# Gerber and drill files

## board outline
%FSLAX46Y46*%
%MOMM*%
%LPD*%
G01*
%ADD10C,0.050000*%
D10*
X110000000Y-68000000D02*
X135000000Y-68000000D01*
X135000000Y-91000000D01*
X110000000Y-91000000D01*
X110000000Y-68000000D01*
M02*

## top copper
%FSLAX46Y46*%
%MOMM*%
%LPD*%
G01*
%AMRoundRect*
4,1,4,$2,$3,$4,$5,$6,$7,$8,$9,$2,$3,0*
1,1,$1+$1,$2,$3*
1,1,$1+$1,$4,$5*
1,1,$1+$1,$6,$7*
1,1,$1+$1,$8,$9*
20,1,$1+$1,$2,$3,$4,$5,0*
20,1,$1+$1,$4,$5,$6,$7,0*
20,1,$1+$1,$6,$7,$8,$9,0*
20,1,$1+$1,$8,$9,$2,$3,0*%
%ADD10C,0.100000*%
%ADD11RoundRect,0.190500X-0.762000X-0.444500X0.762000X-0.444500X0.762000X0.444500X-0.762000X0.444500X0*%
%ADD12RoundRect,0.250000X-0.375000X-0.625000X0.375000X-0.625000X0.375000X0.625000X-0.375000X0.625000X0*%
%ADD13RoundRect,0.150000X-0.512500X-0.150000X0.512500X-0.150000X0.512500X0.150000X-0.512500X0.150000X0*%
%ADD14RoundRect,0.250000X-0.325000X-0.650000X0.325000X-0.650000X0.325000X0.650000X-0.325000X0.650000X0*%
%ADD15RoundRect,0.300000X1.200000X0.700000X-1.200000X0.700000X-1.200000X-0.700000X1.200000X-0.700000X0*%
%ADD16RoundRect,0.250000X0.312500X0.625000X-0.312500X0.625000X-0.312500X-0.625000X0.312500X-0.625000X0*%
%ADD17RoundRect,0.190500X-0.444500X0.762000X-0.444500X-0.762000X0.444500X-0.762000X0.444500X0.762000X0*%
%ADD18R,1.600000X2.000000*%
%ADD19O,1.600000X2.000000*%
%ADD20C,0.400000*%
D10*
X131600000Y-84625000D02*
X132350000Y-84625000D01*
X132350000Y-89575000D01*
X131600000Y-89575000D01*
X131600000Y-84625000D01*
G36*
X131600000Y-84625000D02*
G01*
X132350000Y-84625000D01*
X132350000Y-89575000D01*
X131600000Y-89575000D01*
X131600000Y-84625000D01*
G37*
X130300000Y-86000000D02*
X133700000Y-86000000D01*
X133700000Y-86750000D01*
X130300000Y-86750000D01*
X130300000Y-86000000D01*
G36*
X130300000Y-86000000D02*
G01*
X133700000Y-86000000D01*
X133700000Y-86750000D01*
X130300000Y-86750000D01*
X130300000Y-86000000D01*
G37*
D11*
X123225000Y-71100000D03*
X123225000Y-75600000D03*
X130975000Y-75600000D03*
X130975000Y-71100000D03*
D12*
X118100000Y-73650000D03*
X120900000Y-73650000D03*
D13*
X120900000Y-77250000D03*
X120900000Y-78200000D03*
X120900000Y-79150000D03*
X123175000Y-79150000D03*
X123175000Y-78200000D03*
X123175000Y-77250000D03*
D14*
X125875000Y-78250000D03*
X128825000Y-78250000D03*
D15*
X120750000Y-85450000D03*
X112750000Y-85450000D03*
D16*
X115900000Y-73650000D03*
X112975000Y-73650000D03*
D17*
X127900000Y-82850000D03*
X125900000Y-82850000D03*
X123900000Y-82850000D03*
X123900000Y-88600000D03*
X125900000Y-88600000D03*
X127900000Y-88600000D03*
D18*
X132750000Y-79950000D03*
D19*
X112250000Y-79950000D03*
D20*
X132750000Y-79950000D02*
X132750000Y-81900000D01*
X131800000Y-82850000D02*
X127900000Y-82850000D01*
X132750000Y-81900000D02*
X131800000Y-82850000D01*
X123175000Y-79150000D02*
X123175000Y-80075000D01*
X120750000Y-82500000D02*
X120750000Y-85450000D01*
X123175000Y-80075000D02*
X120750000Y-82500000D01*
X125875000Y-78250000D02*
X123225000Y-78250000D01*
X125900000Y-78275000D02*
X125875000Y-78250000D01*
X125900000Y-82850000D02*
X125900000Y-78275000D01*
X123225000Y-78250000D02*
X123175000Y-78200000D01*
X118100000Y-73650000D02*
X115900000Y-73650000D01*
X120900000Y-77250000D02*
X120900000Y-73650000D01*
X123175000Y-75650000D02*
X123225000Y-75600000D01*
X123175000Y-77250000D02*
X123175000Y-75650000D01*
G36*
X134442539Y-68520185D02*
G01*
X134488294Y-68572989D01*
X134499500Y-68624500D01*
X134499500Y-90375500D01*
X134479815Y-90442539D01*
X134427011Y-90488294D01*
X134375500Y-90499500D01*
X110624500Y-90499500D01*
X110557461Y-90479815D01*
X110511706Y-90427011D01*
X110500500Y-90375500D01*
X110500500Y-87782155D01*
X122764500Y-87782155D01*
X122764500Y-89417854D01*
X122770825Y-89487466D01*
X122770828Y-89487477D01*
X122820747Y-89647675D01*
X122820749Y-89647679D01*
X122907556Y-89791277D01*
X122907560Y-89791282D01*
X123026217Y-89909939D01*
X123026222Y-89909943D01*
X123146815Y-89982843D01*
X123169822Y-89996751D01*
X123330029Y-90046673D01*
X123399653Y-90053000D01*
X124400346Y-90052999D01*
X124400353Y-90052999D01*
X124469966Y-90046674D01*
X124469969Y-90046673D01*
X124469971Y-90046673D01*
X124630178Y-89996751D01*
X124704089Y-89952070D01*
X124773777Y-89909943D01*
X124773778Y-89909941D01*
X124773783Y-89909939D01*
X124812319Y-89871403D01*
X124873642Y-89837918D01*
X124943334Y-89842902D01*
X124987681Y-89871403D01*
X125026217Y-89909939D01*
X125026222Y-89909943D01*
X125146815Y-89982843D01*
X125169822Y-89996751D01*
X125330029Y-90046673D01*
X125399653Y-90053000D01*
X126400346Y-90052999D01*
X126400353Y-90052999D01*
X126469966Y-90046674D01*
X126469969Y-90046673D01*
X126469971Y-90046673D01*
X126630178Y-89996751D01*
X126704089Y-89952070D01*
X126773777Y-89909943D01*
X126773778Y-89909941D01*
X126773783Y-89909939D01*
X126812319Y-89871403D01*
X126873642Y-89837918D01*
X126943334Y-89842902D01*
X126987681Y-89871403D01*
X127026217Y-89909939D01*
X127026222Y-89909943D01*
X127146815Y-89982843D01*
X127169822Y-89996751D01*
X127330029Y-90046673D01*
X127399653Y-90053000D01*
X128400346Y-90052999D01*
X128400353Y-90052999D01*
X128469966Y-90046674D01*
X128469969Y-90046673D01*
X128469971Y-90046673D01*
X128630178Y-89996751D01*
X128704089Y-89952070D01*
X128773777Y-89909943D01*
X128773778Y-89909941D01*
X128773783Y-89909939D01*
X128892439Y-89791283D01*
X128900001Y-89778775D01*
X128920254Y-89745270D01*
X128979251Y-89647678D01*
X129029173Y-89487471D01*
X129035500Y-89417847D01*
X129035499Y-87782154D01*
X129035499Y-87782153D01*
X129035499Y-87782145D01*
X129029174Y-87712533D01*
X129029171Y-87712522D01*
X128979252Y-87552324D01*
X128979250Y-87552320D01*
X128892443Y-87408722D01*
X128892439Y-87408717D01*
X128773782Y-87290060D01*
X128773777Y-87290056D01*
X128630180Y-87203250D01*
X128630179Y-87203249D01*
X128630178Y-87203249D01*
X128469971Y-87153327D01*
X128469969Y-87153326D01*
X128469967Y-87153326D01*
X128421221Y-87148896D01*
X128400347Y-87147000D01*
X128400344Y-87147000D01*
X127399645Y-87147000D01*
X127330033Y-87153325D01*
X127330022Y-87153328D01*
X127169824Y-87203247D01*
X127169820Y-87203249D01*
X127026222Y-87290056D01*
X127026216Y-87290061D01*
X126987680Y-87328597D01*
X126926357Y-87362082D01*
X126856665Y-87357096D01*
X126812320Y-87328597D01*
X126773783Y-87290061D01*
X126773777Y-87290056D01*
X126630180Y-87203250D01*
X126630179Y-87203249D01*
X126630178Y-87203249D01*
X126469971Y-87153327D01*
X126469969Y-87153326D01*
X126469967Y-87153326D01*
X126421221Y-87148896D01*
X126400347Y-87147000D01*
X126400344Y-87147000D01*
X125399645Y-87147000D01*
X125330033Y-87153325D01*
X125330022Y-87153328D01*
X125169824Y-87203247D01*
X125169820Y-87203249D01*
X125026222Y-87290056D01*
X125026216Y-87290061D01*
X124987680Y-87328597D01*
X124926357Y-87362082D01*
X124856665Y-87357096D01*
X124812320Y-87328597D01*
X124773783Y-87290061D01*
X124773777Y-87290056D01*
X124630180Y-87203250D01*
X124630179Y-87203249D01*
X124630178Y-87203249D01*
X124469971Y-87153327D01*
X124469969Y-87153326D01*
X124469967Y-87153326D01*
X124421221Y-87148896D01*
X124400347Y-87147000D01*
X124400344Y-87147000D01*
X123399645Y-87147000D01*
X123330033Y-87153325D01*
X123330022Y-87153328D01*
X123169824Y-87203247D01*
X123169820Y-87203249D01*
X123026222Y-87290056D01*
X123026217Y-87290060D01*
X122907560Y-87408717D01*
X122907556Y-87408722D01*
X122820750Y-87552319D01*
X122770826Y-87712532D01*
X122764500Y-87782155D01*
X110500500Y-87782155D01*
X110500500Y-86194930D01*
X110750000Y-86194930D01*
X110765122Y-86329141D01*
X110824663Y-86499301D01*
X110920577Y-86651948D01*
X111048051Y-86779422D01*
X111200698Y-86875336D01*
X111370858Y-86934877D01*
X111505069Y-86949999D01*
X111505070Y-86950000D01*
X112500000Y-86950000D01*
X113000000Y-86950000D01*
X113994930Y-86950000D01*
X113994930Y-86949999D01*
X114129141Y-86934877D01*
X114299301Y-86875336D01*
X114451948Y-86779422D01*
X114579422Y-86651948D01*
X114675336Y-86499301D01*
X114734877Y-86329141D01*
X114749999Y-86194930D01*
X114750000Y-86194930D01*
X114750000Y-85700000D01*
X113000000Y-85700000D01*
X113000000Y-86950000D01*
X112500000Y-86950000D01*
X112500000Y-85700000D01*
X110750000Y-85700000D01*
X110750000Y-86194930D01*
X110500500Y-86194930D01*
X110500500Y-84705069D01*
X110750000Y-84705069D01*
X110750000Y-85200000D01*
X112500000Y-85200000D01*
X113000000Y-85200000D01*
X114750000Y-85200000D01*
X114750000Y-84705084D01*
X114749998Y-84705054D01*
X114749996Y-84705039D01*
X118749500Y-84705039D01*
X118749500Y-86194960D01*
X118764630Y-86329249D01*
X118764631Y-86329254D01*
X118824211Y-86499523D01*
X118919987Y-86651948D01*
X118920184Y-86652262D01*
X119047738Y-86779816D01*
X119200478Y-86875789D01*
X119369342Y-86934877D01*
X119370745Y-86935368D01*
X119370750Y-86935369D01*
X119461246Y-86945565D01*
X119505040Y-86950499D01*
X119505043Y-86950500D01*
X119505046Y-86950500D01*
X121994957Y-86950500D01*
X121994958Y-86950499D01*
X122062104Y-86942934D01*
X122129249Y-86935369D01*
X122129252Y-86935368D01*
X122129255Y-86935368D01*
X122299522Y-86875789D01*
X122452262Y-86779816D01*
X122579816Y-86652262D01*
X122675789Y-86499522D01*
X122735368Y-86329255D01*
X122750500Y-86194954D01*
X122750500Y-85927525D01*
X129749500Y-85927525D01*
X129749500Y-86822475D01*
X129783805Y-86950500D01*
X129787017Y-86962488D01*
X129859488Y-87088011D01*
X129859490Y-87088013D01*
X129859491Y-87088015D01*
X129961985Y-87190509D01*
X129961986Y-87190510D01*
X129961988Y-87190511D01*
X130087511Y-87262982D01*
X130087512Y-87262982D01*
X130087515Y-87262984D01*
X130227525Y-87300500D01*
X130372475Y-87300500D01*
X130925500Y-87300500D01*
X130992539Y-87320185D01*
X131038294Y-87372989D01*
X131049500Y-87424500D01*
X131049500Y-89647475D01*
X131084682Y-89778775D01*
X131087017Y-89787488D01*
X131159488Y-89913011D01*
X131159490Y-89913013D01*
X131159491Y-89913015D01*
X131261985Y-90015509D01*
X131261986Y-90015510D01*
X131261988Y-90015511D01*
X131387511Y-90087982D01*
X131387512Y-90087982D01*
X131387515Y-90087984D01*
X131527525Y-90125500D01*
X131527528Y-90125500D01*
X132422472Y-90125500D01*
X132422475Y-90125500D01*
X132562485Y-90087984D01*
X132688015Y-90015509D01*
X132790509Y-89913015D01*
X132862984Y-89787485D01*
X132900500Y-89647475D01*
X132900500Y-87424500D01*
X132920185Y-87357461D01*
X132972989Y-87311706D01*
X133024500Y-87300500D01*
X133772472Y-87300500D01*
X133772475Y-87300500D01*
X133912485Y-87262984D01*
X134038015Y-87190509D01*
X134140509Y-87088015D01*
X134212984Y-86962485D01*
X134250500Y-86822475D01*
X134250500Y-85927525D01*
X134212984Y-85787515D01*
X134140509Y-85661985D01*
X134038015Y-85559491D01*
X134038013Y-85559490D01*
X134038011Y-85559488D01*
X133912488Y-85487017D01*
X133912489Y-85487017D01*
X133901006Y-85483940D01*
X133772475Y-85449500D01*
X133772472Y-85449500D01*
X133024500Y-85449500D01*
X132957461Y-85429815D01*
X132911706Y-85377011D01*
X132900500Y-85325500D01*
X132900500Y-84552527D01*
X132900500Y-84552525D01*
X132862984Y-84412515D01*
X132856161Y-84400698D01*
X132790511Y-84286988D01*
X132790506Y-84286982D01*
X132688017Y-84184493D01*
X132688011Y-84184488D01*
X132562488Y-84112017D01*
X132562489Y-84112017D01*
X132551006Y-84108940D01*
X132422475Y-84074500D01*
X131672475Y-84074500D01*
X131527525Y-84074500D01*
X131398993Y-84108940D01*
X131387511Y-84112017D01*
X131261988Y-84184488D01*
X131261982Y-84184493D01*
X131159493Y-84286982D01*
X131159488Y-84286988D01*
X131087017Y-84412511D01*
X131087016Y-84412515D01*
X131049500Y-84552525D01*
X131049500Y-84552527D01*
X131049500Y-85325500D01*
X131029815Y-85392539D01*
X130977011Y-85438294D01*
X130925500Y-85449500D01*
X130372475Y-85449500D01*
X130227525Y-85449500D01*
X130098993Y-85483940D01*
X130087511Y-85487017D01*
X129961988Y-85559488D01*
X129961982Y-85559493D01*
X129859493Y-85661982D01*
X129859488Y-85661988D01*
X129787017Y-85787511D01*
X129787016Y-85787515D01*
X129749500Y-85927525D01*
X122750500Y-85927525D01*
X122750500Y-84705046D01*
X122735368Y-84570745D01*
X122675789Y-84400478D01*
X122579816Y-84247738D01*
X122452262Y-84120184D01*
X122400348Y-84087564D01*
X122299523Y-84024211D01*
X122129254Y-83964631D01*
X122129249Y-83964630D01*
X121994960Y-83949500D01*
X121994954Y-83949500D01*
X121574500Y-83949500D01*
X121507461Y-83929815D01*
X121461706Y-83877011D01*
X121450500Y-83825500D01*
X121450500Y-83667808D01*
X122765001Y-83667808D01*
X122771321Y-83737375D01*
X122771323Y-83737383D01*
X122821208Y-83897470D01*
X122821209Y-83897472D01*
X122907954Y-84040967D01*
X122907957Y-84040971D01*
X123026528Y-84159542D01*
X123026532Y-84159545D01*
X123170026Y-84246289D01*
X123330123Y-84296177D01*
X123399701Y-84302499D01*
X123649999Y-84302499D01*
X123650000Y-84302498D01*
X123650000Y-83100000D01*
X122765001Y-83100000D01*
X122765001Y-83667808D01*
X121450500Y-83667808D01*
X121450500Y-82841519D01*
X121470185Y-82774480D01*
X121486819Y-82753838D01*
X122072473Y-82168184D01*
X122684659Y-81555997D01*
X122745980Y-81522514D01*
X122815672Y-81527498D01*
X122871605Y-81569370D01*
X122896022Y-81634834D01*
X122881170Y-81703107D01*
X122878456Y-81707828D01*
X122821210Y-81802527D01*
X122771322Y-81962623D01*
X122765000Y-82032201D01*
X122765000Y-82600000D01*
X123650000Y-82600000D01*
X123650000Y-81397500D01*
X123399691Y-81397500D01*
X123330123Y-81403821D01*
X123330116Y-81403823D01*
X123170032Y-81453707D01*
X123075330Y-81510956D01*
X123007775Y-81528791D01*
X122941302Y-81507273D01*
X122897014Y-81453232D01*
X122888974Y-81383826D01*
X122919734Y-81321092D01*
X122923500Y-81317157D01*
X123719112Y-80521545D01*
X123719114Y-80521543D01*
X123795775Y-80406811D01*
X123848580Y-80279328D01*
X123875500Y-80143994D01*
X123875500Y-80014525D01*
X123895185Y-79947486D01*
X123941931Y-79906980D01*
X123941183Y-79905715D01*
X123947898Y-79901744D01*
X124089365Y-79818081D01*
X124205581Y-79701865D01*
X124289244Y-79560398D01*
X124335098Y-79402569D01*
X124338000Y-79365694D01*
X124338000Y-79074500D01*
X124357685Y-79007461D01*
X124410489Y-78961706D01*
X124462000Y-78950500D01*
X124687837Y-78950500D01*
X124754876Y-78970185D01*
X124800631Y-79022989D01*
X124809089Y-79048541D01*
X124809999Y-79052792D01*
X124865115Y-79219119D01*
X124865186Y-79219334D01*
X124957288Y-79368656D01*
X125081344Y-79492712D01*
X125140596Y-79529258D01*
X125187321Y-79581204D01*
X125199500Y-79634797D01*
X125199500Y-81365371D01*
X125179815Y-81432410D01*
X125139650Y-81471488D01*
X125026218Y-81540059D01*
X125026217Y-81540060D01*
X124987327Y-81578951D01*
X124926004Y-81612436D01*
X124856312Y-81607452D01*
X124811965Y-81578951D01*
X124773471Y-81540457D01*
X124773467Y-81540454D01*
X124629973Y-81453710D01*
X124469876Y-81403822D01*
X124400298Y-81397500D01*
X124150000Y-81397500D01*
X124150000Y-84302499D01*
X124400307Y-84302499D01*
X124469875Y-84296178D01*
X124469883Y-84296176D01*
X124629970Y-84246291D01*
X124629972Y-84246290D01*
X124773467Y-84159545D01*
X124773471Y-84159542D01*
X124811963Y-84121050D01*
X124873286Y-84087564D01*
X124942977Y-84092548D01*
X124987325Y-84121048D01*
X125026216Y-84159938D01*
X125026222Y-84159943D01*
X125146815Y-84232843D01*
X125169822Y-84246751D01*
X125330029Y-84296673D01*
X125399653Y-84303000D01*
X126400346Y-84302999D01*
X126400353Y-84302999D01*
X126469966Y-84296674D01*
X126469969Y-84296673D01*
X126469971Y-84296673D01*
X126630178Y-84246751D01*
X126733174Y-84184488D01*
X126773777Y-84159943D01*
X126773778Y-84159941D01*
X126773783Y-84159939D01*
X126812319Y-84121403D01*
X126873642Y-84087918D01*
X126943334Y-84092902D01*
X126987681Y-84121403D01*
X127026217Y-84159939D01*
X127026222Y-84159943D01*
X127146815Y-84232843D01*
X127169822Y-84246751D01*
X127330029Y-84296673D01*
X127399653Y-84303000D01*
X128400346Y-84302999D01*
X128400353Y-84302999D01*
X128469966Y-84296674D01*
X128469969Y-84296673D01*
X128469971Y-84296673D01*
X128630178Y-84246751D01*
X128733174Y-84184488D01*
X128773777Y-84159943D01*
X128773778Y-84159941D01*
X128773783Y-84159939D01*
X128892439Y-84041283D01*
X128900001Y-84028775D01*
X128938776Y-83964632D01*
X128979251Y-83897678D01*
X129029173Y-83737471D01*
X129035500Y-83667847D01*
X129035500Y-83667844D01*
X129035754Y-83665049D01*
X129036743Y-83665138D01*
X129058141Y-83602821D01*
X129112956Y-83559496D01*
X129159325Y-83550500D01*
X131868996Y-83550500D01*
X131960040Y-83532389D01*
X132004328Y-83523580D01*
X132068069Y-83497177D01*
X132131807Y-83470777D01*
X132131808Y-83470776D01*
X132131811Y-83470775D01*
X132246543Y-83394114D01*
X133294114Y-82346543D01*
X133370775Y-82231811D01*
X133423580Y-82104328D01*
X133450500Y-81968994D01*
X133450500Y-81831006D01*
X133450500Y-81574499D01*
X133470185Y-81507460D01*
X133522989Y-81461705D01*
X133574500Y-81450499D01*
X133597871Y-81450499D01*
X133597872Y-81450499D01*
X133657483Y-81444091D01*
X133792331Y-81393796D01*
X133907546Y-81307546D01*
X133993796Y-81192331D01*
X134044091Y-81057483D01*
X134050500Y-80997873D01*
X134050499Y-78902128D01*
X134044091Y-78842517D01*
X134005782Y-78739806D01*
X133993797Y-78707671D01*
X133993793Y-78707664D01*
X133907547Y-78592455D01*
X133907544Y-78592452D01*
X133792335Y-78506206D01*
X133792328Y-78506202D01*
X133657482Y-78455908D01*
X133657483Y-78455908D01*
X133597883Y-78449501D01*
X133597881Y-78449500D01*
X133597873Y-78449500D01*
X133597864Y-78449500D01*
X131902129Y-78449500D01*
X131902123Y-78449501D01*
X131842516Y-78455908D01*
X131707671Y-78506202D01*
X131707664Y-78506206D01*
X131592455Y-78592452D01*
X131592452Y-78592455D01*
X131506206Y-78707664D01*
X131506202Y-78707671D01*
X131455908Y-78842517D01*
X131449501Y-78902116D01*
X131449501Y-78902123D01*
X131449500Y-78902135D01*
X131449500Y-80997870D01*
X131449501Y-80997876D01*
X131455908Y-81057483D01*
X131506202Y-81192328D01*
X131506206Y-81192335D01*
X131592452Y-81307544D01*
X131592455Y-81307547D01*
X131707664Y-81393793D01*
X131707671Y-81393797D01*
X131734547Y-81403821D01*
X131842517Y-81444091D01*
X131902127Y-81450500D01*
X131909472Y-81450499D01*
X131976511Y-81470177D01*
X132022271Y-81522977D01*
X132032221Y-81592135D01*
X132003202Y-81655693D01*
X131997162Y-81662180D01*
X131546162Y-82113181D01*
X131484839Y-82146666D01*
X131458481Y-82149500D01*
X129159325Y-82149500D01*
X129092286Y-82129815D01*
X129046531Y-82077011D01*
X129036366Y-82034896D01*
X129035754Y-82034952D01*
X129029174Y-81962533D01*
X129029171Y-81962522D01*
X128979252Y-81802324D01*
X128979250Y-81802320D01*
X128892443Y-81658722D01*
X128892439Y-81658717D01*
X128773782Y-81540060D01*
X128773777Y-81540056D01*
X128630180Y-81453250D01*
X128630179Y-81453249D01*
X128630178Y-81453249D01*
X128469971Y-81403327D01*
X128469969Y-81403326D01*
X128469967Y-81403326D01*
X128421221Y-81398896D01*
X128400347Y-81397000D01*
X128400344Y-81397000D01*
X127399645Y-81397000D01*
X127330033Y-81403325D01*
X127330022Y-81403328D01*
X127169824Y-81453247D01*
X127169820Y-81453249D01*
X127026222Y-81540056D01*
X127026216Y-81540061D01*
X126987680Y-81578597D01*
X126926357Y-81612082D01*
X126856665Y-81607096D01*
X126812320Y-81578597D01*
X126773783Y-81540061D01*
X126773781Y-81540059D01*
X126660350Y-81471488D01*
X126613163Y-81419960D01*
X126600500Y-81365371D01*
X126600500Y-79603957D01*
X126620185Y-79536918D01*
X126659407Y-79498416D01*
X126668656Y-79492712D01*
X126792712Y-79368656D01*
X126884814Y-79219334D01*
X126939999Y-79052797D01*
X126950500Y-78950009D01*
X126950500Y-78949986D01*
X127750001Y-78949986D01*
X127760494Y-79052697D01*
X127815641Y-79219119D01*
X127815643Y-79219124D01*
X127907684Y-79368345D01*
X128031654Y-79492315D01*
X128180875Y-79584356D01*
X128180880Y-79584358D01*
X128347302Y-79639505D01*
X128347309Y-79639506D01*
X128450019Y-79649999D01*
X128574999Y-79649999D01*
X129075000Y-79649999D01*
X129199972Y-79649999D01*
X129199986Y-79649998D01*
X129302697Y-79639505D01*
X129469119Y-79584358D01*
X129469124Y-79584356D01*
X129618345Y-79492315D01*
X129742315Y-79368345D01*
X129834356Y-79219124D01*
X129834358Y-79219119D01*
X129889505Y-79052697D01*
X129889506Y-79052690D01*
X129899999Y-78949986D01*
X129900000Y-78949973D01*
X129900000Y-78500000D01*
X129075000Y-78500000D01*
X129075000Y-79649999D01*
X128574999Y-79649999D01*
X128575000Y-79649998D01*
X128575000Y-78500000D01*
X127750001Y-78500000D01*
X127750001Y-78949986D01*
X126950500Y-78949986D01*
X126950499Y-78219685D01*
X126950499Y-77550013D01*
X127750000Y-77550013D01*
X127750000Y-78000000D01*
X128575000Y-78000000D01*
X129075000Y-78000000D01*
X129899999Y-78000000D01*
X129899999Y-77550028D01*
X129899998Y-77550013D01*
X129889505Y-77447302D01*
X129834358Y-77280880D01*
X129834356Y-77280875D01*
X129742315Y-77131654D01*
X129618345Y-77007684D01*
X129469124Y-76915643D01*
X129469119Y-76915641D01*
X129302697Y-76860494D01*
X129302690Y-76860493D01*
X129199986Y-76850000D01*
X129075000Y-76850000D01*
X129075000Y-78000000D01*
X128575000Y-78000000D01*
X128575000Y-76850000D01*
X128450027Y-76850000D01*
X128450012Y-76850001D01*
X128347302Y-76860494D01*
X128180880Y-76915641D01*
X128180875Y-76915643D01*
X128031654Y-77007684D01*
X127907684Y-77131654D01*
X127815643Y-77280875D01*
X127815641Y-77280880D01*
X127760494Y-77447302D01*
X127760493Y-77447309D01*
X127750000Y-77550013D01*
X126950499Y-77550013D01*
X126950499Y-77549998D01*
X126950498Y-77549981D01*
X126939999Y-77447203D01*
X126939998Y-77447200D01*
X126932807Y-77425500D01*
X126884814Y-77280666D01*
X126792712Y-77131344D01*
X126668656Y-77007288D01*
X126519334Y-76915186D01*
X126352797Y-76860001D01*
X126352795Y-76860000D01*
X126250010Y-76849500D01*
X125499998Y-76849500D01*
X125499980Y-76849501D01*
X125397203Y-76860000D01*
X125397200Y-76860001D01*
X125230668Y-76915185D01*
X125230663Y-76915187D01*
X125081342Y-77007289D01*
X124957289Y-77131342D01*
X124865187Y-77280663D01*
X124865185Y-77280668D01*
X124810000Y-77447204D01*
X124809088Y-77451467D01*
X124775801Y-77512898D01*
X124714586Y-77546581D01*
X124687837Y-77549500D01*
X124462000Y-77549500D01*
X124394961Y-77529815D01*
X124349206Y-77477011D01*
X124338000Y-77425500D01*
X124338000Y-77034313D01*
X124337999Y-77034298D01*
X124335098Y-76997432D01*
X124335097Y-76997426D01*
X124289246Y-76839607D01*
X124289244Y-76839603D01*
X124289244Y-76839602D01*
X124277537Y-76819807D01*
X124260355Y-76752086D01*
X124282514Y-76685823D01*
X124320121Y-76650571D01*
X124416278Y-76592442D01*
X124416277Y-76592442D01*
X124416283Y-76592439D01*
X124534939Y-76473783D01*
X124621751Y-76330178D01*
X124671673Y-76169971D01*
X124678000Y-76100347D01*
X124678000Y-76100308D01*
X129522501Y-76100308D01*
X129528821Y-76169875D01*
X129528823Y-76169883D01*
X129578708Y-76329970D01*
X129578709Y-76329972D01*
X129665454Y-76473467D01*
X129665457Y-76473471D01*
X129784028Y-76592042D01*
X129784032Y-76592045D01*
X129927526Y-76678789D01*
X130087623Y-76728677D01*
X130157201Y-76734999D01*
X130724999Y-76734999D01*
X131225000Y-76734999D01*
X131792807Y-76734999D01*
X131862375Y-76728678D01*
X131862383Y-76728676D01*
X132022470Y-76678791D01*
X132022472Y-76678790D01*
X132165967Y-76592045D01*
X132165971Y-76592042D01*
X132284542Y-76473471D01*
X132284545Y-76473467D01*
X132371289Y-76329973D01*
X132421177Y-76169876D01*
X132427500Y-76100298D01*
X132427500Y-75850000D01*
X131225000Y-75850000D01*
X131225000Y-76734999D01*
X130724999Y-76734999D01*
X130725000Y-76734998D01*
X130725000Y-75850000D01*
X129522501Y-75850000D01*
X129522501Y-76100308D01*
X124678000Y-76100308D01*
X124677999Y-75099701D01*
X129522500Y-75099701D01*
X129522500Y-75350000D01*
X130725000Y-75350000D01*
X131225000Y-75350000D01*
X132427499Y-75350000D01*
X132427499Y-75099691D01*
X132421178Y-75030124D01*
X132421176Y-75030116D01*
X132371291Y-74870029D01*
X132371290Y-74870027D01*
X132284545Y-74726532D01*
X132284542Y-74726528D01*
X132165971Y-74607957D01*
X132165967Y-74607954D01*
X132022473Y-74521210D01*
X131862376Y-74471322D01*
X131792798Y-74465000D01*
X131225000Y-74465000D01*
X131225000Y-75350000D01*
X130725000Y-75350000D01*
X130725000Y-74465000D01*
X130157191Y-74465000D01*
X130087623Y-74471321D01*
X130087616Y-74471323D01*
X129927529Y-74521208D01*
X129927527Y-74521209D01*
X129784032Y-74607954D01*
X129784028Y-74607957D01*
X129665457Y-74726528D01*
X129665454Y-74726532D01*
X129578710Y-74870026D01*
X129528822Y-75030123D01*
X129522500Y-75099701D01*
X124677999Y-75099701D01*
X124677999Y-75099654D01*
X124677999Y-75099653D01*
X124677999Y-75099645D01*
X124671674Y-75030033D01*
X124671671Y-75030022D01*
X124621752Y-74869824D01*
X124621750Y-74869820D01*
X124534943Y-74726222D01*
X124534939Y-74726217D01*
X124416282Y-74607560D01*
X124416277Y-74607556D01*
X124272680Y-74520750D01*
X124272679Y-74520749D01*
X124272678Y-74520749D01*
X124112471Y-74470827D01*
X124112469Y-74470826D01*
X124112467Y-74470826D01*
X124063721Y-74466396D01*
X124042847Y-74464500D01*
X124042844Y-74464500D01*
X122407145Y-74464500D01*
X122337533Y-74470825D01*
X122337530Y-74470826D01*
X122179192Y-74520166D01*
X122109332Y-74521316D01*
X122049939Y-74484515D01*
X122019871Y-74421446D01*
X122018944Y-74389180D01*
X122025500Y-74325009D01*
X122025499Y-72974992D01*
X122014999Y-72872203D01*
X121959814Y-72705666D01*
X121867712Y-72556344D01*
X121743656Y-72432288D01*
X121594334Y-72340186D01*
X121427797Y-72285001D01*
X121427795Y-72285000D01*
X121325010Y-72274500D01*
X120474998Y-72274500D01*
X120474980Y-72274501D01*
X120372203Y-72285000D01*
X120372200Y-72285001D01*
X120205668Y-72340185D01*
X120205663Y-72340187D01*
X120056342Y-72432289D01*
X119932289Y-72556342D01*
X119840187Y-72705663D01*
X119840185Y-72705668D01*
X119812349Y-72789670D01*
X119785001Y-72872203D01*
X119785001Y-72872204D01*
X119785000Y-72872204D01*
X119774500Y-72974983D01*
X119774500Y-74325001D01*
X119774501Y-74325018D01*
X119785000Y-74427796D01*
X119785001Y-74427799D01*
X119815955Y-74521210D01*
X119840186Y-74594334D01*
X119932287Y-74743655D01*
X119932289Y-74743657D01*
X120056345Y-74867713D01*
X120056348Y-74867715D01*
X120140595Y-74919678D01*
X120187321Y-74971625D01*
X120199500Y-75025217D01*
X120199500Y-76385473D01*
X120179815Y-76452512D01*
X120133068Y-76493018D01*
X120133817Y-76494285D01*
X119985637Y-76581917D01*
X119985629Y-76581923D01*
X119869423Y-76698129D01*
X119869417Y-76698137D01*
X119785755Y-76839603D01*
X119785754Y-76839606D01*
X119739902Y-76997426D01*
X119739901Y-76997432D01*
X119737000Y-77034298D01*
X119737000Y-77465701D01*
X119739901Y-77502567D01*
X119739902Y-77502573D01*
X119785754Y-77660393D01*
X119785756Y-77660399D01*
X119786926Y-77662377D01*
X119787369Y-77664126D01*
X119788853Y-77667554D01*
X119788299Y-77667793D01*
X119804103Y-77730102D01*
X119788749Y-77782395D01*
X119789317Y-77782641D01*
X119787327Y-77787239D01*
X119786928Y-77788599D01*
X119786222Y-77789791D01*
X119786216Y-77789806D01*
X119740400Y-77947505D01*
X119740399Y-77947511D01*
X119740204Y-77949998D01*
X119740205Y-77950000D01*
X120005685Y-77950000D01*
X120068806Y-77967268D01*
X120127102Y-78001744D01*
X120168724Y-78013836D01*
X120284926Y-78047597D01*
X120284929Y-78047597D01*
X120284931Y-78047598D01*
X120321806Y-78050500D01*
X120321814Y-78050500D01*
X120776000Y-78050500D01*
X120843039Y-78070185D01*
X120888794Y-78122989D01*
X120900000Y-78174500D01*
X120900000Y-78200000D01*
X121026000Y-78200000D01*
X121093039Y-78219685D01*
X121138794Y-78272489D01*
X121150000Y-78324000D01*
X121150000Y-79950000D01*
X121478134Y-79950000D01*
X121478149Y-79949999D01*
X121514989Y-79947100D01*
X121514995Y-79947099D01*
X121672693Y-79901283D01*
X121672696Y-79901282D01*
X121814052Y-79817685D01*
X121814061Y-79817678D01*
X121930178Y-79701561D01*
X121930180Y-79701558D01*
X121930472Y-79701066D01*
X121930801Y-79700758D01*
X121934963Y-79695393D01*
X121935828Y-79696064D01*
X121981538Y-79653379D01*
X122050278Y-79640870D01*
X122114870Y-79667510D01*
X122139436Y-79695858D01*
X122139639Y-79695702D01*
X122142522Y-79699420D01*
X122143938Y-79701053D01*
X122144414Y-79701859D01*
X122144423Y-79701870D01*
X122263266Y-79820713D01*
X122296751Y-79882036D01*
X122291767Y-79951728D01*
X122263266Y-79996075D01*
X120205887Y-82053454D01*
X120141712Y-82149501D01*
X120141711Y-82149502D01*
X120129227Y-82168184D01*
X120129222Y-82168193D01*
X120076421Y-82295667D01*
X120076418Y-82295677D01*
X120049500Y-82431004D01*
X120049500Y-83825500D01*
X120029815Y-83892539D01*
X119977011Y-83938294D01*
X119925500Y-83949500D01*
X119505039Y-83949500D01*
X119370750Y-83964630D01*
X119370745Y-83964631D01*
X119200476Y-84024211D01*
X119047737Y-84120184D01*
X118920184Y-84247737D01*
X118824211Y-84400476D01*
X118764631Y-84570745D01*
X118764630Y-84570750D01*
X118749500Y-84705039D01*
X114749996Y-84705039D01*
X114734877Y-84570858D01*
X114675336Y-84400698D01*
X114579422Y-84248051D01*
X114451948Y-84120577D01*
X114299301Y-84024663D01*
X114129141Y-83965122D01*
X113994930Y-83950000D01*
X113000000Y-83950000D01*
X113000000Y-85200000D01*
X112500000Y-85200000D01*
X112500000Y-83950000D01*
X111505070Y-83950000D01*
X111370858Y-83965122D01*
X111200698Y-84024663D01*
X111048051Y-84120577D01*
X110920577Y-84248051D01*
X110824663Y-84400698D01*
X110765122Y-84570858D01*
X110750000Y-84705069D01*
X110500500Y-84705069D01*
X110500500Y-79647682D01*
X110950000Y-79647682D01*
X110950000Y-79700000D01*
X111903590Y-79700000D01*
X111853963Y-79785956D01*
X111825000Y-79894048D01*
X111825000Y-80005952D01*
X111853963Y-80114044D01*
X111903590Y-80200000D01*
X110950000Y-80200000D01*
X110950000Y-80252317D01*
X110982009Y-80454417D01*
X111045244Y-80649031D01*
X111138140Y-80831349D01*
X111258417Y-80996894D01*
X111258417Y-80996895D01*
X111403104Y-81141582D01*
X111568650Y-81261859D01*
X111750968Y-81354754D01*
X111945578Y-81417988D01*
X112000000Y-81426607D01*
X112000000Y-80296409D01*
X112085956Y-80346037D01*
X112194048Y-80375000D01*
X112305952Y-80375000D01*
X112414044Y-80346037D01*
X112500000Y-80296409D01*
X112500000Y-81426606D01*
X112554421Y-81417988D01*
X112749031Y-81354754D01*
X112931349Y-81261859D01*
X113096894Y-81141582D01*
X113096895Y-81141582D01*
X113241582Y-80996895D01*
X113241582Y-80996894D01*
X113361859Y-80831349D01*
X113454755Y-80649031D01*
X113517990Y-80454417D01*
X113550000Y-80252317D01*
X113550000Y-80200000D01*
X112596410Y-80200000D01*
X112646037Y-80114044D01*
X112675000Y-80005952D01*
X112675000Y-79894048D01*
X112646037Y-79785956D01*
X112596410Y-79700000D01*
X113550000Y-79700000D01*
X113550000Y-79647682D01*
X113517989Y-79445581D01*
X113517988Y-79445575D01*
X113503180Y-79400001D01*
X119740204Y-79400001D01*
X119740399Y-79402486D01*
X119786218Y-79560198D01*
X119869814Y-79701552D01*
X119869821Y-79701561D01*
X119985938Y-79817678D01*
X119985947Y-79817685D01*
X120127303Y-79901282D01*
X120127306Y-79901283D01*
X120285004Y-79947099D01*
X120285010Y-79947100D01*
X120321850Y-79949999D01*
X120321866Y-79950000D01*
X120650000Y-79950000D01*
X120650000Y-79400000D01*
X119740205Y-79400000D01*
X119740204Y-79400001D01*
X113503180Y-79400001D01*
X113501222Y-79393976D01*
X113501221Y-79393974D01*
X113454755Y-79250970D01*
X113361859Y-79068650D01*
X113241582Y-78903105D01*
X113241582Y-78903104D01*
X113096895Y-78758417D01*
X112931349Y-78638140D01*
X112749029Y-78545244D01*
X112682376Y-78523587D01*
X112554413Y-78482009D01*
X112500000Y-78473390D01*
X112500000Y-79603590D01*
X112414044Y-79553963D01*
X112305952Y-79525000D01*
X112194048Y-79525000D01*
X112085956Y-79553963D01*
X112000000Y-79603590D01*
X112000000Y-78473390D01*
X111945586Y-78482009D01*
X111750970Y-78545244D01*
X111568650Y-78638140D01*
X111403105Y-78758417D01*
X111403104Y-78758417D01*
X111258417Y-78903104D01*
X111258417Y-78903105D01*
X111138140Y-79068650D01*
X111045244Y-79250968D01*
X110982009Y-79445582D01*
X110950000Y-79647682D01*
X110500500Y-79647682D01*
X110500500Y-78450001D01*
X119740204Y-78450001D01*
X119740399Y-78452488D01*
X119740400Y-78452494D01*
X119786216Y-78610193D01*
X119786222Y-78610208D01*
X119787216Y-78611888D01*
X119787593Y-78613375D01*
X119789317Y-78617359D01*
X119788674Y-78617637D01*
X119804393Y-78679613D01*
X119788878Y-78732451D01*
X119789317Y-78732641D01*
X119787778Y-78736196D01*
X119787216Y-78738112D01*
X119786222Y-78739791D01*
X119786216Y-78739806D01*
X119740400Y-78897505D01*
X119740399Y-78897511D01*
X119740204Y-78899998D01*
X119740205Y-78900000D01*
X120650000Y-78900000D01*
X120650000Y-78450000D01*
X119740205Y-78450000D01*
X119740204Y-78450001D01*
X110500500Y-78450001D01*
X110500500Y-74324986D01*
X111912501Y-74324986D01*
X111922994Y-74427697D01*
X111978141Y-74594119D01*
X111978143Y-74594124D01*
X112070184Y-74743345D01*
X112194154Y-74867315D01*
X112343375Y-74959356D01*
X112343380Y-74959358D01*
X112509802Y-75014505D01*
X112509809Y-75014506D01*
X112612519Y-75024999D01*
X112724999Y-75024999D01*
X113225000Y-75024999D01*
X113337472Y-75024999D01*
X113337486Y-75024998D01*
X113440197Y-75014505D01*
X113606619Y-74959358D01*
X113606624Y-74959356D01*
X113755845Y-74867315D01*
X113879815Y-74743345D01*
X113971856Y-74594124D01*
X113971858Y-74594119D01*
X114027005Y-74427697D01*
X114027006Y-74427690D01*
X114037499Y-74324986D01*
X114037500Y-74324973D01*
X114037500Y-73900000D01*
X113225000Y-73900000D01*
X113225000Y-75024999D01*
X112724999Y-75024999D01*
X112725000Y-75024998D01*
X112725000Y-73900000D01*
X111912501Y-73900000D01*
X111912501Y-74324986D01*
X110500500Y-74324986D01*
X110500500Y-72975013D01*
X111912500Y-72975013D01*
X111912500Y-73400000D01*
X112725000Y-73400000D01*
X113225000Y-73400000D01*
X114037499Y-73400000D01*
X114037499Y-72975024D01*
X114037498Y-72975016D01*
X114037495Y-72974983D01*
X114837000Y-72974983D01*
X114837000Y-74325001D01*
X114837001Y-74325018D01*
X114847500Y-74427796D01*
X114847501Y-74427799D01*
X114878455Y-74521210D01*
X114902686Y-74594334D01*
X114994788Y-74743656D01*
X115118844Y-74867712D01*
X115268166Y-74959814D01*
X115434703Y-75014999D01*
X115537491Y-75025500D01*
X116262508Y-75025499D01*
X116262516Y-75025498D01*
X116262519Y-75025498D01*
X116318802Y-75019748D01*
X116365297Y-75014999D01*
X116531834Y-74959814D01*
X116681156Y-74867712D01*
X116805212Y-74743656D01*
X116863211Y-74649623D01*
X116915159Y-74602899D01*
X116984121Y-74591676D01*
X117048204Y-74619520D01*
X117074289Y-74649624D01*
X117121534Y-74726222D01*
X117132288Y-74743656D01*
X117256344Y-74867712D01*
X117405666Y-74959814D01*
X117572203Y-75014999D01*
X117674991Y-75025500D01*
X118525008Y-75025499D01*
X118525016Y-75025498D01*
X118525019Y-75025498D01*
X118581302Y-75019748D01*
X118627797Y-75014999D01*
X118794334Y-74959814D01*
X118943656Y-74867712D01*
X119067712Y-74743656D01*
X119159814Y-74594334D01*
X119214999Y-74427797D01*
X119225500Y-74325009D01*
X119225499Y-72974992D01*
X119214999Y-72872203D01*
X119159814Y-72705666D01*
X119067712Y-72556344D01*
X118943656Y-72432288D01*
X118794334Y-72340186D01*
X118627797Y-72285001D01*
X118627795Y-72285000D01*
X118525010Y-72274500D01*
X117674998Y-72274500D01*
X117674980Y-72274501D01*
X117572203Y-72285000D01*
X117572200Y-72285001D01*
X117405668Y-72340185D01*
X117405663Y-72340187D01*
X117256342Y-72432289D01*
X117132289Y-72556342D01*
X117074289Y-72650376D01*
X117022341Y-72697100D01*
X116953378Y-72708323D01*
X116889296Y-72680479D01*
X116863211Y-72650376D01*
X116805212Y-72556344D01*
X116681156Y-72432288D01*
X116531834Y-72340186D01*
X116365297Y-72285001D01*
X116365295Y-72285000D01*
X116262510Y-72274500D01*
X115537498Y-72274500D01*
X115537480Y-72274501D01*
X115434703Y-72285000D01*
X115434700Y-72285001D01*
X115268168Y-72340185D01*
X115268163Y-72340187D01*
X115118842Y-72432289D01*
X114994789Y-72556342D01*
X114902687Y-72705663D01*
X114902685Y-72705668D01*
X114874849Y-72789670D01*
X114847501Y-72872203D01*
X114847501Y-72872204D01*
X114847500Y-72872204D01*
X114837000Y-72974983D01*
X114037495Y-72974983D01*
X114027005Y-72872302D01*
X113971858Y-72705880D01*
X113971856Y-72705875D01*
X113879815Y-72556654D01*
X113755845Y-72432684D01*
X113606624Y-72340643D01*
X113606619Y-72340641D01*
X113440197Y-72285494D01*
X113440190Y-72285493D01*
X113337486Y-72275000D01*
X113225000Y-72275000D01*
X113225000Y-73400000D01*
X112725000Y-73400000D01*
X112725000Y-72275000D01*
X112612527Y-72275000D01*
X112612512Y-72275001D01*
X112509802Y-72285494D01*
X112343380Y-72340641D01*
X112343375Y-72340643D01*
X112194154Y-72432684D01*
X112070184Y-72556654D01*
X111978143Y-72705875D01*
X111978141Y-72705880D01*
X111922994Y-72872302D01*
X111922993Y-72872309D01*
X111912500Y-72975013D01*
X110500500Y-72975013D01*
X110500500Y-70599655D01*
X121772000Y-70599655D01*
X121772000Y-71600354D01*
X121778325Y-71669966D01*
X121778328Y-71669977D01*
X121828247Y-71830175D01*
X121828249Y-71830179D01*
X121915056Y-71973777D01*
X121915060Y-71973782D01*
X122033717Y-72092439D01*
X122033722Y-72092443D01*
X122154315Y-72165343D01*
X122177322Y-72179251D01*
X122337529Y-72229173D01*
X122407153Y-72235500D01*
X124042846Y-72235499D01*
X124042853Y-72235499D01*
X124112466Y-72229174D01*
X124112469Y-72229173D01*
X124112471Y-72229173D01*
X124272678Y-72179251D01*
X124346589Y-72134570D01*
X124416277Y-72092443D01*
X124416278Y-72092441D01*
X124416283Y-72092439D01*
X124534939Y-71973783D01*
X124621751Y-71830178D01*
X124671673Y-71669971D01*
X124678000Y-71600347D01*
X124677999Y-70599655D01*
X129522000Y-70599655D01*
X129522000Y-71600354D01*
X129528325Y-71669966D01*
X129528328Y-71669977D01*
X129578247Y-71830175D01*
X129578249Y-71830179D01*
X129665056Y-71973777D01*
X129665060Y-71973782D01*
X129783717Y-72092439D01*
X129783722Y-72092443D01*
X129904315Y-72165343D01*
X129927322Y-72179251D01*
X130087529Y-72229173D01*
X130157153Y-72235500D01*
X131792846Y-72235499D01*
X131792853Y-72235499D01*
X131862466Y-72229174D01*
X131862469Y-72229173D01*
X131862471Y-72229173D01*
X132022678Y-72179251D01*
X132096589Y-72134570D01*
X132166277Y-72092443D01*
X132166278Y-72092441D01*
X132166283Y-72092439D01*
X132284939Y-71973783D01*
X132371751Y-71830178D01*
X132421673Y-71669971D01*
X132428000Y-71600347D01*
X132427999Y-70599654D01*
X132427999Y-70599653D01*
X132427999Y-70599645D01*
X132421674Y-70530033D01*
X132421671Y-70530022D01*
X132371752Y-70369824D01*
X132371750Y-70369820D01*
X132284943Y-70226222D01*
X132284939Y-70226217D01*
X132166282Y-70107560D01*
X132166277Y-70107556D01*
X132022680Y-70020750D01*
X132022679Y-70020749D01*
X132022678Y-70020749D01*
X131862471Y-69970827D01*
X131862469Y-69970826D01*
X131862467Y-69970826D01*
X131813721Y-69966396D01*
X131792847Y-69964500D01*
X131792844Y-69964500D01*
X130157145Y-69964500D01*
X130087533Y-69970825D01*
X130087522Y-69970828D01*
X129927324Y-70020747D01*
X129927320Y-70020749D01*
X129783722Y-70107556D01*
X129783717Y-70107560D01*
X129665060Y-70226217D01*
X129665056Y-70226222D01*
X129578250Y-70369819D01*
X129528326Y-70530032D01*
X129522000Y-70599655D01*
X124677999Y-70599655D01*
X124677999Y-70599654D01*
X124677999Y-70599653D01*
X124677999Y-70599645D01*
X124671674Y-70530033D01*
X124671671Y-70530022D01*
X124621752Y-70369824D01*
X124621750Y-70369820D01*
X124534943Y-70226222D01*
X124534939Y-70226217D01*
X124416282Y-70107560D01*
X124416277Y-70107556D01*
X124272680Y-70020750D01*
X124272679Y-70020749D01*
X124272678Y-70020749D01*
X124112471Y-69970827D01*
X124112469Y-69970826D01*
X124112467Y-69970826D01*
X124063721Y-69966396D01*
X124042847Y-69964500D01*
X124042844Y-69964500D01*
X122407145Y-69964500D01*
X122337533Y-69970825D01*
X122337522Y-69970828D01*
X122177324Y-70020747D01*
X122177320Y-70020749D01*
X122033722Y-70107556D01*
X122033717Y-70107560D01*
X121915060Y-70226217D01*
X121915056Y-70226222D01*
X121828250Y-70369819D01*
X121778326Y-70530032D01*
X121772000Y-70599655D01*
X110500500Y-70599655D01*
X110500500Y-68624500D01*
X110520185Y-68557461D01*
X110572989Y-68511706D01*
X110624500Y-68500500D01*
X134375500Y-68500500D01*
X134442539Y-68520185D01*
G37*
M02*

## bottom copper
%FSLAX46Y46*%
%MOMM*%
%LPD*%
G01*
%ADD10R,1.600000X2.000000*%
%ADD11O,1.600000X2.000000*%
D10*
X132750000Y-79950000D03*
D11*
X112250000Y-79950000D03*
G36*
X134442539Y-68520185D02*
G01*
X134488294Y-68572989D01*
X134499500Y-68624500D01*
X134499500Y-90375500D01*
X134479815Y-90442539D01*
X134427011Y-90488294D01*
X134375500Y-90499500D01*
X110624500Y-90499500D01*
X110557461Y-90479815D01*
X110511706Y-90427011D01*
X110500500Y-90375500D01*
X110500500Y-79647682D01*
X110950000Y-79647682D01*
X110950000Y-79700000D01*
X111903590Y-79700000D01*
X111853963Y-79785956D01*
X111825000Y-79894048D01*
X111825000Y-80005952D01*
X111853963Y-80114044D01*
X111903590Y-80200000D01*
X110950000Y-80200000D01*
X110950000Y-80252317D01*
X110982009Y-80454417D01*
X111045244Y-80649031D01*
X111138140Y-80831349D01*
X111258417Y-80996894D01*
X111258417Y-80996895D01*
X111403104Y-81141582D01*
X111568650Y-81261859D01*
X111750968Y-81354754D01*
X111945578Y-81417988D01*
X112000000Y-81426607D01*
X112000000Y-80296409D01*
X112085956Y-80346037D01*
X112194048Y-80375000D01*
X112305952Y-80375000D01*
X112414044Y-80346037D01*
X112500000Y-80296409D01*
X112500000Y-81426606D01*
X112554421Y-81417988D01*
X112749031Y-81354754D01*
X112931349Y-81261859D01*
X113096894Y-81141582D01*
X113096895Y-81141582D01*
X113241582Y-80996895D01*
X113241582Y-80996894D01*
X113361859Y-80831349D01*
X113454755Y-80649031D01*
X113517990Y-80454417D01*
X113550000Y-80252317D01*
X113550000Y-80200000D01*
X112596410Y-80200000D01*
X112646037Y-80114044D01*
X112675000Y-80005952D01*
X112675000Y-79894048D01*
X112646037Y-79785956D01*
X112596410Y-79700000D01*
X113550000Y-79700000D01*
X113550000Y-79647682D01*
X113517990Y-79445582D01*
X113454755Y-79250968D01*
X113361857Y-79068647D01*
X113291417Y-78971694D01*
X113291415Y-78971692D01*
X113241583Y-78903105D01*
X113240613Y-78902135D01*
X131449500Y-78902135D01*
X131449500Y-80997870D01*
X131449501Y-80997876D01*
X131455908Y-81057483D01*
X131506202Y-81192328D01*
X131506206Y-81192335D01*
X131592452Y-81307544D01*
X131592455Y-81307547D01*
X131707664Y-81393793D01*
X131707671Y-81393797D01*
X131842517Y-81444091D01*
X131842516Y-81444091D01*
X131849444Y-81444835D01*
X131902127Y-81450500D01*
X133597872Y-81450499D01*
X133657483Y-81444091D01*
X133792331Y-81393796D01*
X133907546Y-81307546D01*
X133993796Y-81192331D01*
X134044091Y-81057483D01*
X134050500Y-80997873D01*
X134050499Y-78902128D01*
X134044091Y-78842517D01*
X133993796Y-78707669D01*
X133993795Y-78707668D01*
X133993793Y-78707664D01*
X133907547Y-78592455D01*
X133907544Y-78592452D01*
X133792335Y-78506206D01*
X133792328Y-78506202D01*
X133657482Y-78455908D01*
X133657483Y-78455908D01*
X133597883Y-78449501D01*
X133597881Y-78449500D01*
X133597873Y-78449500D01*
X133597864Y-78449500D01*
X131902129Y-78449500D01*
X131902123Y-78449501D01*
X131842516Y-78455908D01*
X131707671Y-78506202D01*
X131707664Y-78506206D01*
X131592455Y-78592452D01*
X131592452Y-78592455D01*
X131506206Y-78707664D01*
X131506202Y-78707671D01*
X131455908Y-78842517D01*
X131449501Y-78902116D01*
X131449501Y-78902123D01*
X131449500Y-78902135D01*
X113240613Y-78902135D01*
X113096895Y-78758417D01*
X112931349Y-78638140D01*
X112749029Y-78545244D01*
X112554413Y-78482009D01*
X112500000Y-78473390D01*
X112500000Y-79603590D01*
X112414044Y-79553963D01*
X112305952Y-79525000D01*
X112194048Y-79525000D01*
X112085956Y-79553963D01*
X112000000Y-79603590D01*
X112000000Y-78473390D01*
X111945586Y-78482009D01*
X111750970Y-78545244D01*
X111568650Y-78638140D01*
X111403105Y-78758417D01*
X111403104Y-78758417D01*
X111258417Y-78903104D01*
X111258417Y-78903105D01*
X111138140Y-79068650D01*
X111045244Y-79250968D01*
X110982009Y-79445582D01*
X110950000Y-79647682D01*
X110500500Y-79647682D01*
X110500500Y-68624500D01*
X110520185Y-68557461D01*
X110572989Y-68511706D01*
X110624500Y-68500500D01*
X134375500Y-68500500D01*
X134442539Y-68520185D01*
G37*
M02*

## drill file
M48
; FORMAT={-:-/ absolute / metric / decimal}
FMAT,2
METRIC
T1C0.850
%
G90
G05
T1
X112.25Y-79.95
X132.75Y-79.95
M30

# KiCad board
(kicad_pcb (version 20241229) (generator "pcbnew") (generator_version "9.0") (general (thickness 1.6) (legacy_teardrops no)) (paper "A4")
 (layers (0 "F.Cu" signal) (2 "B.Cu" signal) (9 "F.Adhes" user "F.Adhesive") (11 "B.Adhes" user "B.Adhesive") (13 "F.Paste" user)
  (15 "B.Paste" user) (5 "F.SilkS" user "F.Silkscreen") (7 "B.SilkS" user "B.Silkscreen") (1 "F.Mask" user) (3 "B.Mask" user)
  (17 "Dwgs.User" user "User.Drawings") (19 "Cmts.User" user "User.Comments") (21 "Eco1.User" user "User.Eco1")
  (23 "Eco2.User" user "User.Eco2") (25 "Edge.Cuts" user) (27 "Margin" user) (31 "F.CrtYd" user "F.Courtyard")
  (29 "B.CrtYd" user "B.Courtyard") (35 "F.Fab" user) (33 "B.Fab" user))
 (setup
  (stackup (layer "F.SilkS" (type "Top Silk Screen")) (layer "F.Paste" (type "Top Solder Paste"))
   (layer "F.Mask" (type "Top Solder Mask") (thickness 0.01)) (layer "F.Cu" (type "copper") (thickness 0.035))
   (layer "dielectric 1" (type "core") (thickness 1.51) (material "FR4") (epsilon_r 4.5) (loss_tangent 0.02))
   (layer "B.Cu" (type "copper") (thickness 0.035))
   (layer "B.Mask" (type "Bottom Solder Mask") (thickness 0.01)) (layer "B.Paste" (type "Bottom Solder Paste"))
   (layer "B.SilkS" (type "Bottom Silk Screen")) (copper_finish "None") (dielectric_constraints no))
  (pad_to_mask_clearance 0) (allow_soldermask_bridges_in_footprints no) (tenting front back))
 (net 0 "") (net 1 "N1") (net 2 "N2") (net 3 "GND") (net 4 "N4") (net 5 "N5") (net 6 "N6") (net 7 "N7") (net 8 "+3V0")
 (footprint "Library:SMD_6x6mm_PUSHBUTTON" (layer "F.Cu") (at 127.225 73.6)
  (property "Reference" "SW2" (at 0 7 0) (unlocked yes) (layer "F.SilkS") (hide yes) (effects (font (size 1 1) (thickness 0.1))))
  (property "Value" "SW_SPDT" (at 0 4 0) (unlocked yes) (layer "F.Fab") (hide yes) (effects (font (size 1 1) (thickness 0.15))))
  (pad "1" smd roundrect (at -4 -2.5) (size 1.905 1.27) (layers "F.Cu" "F.Mask" "F.Paste") (roundrect_rratio 0.15) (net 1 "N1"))
  (pad "2" smd roundrect (at -4 2) (size 1.905 1.27) (layers "F.Cu" "F.Mask" "F.Paste") (roundrect_rratio 0.15) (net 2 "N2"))
  (pad "3" smd roundrect (at 3.75 2) (size 1.905 1.27) (layers "F.Cu" "F.Mask" "F.Paste") (roundrect_rratio 0.15) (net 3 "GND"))
  (pad "4" smd roundrect (at 3.75 -2.5) (size 1.905 1.27) (layers "F.Cu" "F.Mask" "F.Paste") (roundrect_rratio 0.15))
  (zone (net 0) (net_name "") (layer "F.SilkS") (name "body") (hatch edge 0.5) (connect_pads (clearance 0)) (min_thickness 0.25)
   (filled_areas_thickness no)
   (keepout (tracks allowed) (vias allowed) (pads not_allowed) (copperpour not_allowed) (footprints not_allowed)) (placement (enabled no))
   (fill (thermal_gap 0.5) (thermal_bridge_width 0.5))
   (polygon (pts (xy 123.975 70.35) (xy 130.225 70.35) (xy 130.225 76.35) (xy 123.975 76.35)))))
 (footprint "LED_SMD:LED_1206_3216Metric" (layer "F.Cu") (at 119.5 73.65)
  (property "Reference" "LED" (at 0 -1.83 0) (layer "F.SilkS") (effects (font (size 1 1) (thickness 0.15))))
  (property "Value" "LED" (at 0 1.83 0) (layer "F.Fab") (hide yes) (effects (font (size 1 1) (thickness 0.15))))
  (pad "1" smd roundrect (at -1.4 0) (size 1.25 1.75) (layers "F.Cu" "F.Mask" "F.Paste") (roundrect_rratio 0.2) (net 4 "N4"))
  (pad "2" smd roundrect (at 1.4 0) (size 1.25 1.75) (layers "F.Cu" "F.Mask" "F.Paste") (roundrect_rratio 0.2) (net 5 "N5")))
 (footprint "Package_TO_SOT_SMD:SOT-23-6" (layer "F.Cu") (at 122.0375 78.2)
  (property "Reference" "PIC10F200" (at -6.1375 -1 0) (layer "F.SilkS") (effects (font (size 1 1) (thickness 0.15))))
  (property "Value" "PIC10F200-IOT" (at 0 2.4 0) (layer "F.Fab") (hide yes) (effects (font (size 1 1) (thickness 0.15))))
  (pad "1" smd roundrect (at -1.1375 -0.95) (size 1.325 0.6) (layers "F.Cu" "F.Mask" "F.Paste") (roundrect_rratio 0.25) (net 5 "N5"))
  (pad "2" smd roundrect (at -1.1375 0) (size 1.325 0.6) (layers "F.Cu" "F.Mask" "F.Paste") (roundrect_rratio 0.25) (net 3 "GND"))
  (pad "3" smd roundrect (at -1.1375 0.95) (size 1.325 0.6) (layers "F.Cu" "F.Mask" "F.Paste") (roundrect_rratio 0.25) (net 3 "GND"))
  (pad "4" smd roundrect (at 1.1375 0.95) (size 1.325 0.6) (layers "F.Cu" "F.Mask" "F.Paste") (roundrect_rratio 0.25) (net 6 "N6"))
  (pad "5" smd roundrect (at 1.1375 0) (size 1.325 0.6) (layers "F.Cu" "F.Mask" "F.Paste") (roundrect_rratio 0.25) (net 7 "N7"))
  (pad "6" smd roundrect (at 1.1375 -0.95) (size 1.325 0.6) (layers "F.Cu" "F.Mask" "F.Paste") (roundrect_rratio 0.25) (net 2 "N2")))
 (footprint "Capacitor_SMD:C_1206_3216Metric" (layer "F.Cu") (at 127.35 78.25)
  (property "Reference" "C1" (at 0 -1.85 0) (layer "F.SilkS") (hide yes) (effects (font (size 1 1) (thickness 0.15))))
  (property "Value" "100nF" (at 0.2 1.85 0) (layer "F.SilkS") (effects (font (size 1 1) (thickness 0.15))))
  (pad "1" smd roundrect (at -1.475 0) (size 1.15 1.8) (layers "F.Cu" "F.Mask" "F.Paste") (roundrect_rratio 0.217391) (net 7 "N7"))
  (pad "2" smd roundrect (at 1.475 0) (size 1.15 1.8) (layers "F.Cu" "F.Mask" "F.Paste") (roundrect_rratio 0.217391) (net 3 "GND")))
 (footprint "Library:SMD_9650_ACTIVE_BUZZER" (layer "F.Cu") (at 116.25 80.45 180)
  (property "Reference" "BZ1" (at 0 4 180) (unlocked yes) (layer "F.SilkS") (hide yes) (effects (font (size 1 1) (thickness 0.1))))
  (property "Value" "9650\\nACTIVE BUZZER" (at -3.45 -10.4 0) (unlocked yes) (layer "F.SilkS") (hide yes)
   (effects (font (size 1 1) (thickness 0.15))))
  (pad "1" smd roundrect (at -4.5 -5 180) (size 3 2) (layers "F.Cu" "F.Mask" "F.Paste") (roundrect_rratio 0.15) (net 6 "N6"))
  (pad "2" smd roundrect (at 3.5 -5 180) (size 3 2) (layers "F.Cu" "F.Mask" "F.Paste") (roundrect_rratio 0.15) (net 3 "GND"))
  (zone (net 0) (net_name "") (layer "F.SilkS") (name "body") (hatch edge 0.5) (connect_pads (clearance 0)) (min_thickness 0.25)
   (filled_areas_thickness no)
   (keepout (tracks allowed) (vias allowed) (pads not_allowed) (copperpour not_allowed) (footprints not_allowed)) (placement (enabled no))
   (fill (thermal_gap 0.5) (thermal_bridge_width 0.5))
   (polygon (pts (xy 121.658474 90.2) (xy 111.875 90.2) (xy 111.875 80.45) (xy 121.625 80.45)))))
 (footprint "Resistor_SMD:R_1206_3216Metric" (layer "F.Cu") (at 114.4375 73.65 180)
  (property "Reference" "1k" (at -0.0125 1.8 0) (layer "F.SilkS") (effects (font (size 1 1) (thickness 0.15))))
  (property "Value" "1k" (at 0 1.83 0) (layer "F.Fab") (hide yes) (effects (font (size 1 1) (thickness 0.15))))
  (pad "1" smd roundrect (at -1.4625 0 180) (size 1.125 1.75) (layers "F.Cu" "F.Mask" "F.Paste") (roundrect_rratio 0.222222) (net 4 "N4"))
  (pad "2" smd roundrect (at 1.4625 0 180) (size 1.125 1.75) (layers "F.Cu" "F.Mask" "F.Paste") (roundrect_rratio 0.222222) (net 3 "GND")))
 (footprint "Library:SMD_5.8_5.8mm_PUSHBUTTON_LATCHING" (layer "F.Cu") (at 125.9 85.85 -90)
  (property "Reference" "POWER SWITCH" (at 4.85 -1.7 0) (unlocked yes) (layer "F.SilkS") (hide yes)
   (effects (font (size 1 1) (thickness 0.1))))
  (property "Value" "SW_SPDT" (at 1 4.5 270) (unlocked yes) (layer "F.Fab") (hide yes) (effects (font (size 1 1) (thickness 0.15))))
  (pad "1" smd roundrect (at -3 -2 270) (size 1.905 1.27) (layers "F.Cu" "F.Mask" "F.Paste") (roundrect_rratio 0.15) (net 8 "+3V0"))
  (pad "2" smd roundrect (at -3 0 270) (size 1.905 1.27) (layers "F.Cu" "F.Mask" "F.Paste") (roundrect_rratio 0.15) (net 7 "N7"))
  (pad "3" smd roundrect (at -3 2 270) (size 1.905 1.27) (layers "F.Cu" "F.Mask" "F.Paste") (roundrect_rratio 0.15) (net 3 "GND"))
  (pad "4" smd roundrect (at 2.75 2 270) (size 1.905 1.27) (layers "F.Cu" "F.Mask" "F.Paste") (roundrect_rratio 0.15))
  (pad "5" smd roundrect (at 2.75 0 270) (size 1.905 1.27) (layers "F.Cu" "F.Mask" "F.Paste") (roundrect_rratio 0.15))
  (pad "6" smd roundrect (at 2.75 -2 270) (size 1.905 1.27) (layers "F.Cu" "F.Mask" "F.Paste") (roundrect_rratio 0.15))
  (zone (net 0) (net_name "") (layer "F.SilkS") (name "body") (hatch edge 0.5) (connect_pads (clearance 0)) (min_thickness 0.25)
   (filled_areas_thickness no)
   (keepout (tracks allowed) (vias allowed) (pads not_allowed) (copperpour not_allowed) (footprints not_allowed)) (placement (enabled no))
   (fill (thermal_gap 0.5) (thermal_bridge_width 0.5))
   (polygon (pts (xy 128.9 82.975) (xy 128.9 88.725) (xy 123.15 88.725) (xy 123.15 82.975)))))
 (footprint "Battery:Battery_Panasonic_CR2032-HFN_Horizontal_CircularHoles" (layer "B.Cu") (at 132.75 79.95 180)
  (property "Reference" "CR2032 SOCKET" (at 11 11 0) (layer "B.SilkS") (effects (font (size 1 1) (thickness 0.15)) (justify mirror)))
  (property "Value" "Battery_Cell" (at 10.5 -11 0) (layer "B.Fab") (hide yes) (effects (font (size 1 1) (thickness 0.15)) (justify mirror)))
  (pad "1" thru_hole rect (at 0 0 180) (size 1.6 2) (drill 0.85) (layers "*.Cu" "*.Mask") (remove_unused_layers no) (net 8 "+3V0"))
  (pad "2" thru_hole oval (at 20.5 0 180) (size 1.6 2) (drill 0.85) (layers "*.Cu" "*.Mask") (remove_unused_layers no) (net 3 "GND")))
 (gr_rect (start 131.6 84.625) (end 132.35 89.575) (stroke (width 0.1) (type solid)) (fill yes) (layer "F.Cu"))
 (gr_rect (start 130.3 86) (end 133.7 86.75) (stroke (width 0.1) (type solid)) (fill yes) (layer "F.Cu"))
 (gr_rect (start 110 68) (end 135 91) (stroke (width 0.05) (type default)) (fill no) (layer "Edge.Cuts"))
 (segment (start 132.75 79.95) (end 132.75 81.9) (width 0.4) (layer "F.Cu") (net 8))
 (segment (start 131.8 82.85) (end 127.9 82.85) (width 0.4) (layer "F.Cu") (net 8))
 (segment (start 132.75 81.9) (end 131.8 82.85) (width 0.4) (layer "F.Cu") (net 8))
 (segment (start 123.175 79.15) (end 123.175 80.075) (width 0.4) (layer "F.Cu") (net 6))
 (segment (start 120.75 82.5) (end 120.75 85.45) (width 0.4) (layer "F.Cu") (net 6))
 (segment (start 123.175 80.075) (end 120.75 82.5) (width 0.4) (layer "F.Cu") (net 6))
 (segment (start 125.875 78.25) (end 123.225 78.25) (width 0.4) (layer "F.Cu") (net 7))
 (segment (start 125.9 78.275) (end 125.875 78.25) (width 0.4) (layer "F.Cu") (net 7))
 (segment (start 125.9 82.85) (end 125.9 78.275) (width 0.4) (layer "F.Cu") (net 7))
 (segment (start 123.225 78.25) (end 123.175 78.2) (width 0.4) (layer "F.Cu") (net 7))
 (segment (start 118.1 73.65) (end 115.9 73.65) (width 0.4) (layer "F.Cu") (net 4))
 (segment (start 120.9 77.25) (end 120.9 73.65) (width 0.4) (layer "F.Cu") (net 5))
 (segment (start 123.175 75.65) (end 123.225 75.6) (width 0.4) (layer "F.Cu") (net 2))
 (segment (start 123.175 77.25) (end 123.175 75.65) (width 0.4) (layer "F.Cu") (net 2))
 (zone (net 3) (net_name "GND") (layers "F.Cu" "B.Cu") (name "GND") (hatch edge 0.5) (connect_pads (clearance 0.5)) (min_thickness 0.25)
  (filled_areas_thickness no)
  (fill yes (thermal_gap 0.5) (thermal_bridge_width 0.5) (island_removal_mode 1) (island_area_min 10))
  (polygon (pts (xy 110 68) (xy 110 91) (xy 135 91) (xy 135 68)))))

